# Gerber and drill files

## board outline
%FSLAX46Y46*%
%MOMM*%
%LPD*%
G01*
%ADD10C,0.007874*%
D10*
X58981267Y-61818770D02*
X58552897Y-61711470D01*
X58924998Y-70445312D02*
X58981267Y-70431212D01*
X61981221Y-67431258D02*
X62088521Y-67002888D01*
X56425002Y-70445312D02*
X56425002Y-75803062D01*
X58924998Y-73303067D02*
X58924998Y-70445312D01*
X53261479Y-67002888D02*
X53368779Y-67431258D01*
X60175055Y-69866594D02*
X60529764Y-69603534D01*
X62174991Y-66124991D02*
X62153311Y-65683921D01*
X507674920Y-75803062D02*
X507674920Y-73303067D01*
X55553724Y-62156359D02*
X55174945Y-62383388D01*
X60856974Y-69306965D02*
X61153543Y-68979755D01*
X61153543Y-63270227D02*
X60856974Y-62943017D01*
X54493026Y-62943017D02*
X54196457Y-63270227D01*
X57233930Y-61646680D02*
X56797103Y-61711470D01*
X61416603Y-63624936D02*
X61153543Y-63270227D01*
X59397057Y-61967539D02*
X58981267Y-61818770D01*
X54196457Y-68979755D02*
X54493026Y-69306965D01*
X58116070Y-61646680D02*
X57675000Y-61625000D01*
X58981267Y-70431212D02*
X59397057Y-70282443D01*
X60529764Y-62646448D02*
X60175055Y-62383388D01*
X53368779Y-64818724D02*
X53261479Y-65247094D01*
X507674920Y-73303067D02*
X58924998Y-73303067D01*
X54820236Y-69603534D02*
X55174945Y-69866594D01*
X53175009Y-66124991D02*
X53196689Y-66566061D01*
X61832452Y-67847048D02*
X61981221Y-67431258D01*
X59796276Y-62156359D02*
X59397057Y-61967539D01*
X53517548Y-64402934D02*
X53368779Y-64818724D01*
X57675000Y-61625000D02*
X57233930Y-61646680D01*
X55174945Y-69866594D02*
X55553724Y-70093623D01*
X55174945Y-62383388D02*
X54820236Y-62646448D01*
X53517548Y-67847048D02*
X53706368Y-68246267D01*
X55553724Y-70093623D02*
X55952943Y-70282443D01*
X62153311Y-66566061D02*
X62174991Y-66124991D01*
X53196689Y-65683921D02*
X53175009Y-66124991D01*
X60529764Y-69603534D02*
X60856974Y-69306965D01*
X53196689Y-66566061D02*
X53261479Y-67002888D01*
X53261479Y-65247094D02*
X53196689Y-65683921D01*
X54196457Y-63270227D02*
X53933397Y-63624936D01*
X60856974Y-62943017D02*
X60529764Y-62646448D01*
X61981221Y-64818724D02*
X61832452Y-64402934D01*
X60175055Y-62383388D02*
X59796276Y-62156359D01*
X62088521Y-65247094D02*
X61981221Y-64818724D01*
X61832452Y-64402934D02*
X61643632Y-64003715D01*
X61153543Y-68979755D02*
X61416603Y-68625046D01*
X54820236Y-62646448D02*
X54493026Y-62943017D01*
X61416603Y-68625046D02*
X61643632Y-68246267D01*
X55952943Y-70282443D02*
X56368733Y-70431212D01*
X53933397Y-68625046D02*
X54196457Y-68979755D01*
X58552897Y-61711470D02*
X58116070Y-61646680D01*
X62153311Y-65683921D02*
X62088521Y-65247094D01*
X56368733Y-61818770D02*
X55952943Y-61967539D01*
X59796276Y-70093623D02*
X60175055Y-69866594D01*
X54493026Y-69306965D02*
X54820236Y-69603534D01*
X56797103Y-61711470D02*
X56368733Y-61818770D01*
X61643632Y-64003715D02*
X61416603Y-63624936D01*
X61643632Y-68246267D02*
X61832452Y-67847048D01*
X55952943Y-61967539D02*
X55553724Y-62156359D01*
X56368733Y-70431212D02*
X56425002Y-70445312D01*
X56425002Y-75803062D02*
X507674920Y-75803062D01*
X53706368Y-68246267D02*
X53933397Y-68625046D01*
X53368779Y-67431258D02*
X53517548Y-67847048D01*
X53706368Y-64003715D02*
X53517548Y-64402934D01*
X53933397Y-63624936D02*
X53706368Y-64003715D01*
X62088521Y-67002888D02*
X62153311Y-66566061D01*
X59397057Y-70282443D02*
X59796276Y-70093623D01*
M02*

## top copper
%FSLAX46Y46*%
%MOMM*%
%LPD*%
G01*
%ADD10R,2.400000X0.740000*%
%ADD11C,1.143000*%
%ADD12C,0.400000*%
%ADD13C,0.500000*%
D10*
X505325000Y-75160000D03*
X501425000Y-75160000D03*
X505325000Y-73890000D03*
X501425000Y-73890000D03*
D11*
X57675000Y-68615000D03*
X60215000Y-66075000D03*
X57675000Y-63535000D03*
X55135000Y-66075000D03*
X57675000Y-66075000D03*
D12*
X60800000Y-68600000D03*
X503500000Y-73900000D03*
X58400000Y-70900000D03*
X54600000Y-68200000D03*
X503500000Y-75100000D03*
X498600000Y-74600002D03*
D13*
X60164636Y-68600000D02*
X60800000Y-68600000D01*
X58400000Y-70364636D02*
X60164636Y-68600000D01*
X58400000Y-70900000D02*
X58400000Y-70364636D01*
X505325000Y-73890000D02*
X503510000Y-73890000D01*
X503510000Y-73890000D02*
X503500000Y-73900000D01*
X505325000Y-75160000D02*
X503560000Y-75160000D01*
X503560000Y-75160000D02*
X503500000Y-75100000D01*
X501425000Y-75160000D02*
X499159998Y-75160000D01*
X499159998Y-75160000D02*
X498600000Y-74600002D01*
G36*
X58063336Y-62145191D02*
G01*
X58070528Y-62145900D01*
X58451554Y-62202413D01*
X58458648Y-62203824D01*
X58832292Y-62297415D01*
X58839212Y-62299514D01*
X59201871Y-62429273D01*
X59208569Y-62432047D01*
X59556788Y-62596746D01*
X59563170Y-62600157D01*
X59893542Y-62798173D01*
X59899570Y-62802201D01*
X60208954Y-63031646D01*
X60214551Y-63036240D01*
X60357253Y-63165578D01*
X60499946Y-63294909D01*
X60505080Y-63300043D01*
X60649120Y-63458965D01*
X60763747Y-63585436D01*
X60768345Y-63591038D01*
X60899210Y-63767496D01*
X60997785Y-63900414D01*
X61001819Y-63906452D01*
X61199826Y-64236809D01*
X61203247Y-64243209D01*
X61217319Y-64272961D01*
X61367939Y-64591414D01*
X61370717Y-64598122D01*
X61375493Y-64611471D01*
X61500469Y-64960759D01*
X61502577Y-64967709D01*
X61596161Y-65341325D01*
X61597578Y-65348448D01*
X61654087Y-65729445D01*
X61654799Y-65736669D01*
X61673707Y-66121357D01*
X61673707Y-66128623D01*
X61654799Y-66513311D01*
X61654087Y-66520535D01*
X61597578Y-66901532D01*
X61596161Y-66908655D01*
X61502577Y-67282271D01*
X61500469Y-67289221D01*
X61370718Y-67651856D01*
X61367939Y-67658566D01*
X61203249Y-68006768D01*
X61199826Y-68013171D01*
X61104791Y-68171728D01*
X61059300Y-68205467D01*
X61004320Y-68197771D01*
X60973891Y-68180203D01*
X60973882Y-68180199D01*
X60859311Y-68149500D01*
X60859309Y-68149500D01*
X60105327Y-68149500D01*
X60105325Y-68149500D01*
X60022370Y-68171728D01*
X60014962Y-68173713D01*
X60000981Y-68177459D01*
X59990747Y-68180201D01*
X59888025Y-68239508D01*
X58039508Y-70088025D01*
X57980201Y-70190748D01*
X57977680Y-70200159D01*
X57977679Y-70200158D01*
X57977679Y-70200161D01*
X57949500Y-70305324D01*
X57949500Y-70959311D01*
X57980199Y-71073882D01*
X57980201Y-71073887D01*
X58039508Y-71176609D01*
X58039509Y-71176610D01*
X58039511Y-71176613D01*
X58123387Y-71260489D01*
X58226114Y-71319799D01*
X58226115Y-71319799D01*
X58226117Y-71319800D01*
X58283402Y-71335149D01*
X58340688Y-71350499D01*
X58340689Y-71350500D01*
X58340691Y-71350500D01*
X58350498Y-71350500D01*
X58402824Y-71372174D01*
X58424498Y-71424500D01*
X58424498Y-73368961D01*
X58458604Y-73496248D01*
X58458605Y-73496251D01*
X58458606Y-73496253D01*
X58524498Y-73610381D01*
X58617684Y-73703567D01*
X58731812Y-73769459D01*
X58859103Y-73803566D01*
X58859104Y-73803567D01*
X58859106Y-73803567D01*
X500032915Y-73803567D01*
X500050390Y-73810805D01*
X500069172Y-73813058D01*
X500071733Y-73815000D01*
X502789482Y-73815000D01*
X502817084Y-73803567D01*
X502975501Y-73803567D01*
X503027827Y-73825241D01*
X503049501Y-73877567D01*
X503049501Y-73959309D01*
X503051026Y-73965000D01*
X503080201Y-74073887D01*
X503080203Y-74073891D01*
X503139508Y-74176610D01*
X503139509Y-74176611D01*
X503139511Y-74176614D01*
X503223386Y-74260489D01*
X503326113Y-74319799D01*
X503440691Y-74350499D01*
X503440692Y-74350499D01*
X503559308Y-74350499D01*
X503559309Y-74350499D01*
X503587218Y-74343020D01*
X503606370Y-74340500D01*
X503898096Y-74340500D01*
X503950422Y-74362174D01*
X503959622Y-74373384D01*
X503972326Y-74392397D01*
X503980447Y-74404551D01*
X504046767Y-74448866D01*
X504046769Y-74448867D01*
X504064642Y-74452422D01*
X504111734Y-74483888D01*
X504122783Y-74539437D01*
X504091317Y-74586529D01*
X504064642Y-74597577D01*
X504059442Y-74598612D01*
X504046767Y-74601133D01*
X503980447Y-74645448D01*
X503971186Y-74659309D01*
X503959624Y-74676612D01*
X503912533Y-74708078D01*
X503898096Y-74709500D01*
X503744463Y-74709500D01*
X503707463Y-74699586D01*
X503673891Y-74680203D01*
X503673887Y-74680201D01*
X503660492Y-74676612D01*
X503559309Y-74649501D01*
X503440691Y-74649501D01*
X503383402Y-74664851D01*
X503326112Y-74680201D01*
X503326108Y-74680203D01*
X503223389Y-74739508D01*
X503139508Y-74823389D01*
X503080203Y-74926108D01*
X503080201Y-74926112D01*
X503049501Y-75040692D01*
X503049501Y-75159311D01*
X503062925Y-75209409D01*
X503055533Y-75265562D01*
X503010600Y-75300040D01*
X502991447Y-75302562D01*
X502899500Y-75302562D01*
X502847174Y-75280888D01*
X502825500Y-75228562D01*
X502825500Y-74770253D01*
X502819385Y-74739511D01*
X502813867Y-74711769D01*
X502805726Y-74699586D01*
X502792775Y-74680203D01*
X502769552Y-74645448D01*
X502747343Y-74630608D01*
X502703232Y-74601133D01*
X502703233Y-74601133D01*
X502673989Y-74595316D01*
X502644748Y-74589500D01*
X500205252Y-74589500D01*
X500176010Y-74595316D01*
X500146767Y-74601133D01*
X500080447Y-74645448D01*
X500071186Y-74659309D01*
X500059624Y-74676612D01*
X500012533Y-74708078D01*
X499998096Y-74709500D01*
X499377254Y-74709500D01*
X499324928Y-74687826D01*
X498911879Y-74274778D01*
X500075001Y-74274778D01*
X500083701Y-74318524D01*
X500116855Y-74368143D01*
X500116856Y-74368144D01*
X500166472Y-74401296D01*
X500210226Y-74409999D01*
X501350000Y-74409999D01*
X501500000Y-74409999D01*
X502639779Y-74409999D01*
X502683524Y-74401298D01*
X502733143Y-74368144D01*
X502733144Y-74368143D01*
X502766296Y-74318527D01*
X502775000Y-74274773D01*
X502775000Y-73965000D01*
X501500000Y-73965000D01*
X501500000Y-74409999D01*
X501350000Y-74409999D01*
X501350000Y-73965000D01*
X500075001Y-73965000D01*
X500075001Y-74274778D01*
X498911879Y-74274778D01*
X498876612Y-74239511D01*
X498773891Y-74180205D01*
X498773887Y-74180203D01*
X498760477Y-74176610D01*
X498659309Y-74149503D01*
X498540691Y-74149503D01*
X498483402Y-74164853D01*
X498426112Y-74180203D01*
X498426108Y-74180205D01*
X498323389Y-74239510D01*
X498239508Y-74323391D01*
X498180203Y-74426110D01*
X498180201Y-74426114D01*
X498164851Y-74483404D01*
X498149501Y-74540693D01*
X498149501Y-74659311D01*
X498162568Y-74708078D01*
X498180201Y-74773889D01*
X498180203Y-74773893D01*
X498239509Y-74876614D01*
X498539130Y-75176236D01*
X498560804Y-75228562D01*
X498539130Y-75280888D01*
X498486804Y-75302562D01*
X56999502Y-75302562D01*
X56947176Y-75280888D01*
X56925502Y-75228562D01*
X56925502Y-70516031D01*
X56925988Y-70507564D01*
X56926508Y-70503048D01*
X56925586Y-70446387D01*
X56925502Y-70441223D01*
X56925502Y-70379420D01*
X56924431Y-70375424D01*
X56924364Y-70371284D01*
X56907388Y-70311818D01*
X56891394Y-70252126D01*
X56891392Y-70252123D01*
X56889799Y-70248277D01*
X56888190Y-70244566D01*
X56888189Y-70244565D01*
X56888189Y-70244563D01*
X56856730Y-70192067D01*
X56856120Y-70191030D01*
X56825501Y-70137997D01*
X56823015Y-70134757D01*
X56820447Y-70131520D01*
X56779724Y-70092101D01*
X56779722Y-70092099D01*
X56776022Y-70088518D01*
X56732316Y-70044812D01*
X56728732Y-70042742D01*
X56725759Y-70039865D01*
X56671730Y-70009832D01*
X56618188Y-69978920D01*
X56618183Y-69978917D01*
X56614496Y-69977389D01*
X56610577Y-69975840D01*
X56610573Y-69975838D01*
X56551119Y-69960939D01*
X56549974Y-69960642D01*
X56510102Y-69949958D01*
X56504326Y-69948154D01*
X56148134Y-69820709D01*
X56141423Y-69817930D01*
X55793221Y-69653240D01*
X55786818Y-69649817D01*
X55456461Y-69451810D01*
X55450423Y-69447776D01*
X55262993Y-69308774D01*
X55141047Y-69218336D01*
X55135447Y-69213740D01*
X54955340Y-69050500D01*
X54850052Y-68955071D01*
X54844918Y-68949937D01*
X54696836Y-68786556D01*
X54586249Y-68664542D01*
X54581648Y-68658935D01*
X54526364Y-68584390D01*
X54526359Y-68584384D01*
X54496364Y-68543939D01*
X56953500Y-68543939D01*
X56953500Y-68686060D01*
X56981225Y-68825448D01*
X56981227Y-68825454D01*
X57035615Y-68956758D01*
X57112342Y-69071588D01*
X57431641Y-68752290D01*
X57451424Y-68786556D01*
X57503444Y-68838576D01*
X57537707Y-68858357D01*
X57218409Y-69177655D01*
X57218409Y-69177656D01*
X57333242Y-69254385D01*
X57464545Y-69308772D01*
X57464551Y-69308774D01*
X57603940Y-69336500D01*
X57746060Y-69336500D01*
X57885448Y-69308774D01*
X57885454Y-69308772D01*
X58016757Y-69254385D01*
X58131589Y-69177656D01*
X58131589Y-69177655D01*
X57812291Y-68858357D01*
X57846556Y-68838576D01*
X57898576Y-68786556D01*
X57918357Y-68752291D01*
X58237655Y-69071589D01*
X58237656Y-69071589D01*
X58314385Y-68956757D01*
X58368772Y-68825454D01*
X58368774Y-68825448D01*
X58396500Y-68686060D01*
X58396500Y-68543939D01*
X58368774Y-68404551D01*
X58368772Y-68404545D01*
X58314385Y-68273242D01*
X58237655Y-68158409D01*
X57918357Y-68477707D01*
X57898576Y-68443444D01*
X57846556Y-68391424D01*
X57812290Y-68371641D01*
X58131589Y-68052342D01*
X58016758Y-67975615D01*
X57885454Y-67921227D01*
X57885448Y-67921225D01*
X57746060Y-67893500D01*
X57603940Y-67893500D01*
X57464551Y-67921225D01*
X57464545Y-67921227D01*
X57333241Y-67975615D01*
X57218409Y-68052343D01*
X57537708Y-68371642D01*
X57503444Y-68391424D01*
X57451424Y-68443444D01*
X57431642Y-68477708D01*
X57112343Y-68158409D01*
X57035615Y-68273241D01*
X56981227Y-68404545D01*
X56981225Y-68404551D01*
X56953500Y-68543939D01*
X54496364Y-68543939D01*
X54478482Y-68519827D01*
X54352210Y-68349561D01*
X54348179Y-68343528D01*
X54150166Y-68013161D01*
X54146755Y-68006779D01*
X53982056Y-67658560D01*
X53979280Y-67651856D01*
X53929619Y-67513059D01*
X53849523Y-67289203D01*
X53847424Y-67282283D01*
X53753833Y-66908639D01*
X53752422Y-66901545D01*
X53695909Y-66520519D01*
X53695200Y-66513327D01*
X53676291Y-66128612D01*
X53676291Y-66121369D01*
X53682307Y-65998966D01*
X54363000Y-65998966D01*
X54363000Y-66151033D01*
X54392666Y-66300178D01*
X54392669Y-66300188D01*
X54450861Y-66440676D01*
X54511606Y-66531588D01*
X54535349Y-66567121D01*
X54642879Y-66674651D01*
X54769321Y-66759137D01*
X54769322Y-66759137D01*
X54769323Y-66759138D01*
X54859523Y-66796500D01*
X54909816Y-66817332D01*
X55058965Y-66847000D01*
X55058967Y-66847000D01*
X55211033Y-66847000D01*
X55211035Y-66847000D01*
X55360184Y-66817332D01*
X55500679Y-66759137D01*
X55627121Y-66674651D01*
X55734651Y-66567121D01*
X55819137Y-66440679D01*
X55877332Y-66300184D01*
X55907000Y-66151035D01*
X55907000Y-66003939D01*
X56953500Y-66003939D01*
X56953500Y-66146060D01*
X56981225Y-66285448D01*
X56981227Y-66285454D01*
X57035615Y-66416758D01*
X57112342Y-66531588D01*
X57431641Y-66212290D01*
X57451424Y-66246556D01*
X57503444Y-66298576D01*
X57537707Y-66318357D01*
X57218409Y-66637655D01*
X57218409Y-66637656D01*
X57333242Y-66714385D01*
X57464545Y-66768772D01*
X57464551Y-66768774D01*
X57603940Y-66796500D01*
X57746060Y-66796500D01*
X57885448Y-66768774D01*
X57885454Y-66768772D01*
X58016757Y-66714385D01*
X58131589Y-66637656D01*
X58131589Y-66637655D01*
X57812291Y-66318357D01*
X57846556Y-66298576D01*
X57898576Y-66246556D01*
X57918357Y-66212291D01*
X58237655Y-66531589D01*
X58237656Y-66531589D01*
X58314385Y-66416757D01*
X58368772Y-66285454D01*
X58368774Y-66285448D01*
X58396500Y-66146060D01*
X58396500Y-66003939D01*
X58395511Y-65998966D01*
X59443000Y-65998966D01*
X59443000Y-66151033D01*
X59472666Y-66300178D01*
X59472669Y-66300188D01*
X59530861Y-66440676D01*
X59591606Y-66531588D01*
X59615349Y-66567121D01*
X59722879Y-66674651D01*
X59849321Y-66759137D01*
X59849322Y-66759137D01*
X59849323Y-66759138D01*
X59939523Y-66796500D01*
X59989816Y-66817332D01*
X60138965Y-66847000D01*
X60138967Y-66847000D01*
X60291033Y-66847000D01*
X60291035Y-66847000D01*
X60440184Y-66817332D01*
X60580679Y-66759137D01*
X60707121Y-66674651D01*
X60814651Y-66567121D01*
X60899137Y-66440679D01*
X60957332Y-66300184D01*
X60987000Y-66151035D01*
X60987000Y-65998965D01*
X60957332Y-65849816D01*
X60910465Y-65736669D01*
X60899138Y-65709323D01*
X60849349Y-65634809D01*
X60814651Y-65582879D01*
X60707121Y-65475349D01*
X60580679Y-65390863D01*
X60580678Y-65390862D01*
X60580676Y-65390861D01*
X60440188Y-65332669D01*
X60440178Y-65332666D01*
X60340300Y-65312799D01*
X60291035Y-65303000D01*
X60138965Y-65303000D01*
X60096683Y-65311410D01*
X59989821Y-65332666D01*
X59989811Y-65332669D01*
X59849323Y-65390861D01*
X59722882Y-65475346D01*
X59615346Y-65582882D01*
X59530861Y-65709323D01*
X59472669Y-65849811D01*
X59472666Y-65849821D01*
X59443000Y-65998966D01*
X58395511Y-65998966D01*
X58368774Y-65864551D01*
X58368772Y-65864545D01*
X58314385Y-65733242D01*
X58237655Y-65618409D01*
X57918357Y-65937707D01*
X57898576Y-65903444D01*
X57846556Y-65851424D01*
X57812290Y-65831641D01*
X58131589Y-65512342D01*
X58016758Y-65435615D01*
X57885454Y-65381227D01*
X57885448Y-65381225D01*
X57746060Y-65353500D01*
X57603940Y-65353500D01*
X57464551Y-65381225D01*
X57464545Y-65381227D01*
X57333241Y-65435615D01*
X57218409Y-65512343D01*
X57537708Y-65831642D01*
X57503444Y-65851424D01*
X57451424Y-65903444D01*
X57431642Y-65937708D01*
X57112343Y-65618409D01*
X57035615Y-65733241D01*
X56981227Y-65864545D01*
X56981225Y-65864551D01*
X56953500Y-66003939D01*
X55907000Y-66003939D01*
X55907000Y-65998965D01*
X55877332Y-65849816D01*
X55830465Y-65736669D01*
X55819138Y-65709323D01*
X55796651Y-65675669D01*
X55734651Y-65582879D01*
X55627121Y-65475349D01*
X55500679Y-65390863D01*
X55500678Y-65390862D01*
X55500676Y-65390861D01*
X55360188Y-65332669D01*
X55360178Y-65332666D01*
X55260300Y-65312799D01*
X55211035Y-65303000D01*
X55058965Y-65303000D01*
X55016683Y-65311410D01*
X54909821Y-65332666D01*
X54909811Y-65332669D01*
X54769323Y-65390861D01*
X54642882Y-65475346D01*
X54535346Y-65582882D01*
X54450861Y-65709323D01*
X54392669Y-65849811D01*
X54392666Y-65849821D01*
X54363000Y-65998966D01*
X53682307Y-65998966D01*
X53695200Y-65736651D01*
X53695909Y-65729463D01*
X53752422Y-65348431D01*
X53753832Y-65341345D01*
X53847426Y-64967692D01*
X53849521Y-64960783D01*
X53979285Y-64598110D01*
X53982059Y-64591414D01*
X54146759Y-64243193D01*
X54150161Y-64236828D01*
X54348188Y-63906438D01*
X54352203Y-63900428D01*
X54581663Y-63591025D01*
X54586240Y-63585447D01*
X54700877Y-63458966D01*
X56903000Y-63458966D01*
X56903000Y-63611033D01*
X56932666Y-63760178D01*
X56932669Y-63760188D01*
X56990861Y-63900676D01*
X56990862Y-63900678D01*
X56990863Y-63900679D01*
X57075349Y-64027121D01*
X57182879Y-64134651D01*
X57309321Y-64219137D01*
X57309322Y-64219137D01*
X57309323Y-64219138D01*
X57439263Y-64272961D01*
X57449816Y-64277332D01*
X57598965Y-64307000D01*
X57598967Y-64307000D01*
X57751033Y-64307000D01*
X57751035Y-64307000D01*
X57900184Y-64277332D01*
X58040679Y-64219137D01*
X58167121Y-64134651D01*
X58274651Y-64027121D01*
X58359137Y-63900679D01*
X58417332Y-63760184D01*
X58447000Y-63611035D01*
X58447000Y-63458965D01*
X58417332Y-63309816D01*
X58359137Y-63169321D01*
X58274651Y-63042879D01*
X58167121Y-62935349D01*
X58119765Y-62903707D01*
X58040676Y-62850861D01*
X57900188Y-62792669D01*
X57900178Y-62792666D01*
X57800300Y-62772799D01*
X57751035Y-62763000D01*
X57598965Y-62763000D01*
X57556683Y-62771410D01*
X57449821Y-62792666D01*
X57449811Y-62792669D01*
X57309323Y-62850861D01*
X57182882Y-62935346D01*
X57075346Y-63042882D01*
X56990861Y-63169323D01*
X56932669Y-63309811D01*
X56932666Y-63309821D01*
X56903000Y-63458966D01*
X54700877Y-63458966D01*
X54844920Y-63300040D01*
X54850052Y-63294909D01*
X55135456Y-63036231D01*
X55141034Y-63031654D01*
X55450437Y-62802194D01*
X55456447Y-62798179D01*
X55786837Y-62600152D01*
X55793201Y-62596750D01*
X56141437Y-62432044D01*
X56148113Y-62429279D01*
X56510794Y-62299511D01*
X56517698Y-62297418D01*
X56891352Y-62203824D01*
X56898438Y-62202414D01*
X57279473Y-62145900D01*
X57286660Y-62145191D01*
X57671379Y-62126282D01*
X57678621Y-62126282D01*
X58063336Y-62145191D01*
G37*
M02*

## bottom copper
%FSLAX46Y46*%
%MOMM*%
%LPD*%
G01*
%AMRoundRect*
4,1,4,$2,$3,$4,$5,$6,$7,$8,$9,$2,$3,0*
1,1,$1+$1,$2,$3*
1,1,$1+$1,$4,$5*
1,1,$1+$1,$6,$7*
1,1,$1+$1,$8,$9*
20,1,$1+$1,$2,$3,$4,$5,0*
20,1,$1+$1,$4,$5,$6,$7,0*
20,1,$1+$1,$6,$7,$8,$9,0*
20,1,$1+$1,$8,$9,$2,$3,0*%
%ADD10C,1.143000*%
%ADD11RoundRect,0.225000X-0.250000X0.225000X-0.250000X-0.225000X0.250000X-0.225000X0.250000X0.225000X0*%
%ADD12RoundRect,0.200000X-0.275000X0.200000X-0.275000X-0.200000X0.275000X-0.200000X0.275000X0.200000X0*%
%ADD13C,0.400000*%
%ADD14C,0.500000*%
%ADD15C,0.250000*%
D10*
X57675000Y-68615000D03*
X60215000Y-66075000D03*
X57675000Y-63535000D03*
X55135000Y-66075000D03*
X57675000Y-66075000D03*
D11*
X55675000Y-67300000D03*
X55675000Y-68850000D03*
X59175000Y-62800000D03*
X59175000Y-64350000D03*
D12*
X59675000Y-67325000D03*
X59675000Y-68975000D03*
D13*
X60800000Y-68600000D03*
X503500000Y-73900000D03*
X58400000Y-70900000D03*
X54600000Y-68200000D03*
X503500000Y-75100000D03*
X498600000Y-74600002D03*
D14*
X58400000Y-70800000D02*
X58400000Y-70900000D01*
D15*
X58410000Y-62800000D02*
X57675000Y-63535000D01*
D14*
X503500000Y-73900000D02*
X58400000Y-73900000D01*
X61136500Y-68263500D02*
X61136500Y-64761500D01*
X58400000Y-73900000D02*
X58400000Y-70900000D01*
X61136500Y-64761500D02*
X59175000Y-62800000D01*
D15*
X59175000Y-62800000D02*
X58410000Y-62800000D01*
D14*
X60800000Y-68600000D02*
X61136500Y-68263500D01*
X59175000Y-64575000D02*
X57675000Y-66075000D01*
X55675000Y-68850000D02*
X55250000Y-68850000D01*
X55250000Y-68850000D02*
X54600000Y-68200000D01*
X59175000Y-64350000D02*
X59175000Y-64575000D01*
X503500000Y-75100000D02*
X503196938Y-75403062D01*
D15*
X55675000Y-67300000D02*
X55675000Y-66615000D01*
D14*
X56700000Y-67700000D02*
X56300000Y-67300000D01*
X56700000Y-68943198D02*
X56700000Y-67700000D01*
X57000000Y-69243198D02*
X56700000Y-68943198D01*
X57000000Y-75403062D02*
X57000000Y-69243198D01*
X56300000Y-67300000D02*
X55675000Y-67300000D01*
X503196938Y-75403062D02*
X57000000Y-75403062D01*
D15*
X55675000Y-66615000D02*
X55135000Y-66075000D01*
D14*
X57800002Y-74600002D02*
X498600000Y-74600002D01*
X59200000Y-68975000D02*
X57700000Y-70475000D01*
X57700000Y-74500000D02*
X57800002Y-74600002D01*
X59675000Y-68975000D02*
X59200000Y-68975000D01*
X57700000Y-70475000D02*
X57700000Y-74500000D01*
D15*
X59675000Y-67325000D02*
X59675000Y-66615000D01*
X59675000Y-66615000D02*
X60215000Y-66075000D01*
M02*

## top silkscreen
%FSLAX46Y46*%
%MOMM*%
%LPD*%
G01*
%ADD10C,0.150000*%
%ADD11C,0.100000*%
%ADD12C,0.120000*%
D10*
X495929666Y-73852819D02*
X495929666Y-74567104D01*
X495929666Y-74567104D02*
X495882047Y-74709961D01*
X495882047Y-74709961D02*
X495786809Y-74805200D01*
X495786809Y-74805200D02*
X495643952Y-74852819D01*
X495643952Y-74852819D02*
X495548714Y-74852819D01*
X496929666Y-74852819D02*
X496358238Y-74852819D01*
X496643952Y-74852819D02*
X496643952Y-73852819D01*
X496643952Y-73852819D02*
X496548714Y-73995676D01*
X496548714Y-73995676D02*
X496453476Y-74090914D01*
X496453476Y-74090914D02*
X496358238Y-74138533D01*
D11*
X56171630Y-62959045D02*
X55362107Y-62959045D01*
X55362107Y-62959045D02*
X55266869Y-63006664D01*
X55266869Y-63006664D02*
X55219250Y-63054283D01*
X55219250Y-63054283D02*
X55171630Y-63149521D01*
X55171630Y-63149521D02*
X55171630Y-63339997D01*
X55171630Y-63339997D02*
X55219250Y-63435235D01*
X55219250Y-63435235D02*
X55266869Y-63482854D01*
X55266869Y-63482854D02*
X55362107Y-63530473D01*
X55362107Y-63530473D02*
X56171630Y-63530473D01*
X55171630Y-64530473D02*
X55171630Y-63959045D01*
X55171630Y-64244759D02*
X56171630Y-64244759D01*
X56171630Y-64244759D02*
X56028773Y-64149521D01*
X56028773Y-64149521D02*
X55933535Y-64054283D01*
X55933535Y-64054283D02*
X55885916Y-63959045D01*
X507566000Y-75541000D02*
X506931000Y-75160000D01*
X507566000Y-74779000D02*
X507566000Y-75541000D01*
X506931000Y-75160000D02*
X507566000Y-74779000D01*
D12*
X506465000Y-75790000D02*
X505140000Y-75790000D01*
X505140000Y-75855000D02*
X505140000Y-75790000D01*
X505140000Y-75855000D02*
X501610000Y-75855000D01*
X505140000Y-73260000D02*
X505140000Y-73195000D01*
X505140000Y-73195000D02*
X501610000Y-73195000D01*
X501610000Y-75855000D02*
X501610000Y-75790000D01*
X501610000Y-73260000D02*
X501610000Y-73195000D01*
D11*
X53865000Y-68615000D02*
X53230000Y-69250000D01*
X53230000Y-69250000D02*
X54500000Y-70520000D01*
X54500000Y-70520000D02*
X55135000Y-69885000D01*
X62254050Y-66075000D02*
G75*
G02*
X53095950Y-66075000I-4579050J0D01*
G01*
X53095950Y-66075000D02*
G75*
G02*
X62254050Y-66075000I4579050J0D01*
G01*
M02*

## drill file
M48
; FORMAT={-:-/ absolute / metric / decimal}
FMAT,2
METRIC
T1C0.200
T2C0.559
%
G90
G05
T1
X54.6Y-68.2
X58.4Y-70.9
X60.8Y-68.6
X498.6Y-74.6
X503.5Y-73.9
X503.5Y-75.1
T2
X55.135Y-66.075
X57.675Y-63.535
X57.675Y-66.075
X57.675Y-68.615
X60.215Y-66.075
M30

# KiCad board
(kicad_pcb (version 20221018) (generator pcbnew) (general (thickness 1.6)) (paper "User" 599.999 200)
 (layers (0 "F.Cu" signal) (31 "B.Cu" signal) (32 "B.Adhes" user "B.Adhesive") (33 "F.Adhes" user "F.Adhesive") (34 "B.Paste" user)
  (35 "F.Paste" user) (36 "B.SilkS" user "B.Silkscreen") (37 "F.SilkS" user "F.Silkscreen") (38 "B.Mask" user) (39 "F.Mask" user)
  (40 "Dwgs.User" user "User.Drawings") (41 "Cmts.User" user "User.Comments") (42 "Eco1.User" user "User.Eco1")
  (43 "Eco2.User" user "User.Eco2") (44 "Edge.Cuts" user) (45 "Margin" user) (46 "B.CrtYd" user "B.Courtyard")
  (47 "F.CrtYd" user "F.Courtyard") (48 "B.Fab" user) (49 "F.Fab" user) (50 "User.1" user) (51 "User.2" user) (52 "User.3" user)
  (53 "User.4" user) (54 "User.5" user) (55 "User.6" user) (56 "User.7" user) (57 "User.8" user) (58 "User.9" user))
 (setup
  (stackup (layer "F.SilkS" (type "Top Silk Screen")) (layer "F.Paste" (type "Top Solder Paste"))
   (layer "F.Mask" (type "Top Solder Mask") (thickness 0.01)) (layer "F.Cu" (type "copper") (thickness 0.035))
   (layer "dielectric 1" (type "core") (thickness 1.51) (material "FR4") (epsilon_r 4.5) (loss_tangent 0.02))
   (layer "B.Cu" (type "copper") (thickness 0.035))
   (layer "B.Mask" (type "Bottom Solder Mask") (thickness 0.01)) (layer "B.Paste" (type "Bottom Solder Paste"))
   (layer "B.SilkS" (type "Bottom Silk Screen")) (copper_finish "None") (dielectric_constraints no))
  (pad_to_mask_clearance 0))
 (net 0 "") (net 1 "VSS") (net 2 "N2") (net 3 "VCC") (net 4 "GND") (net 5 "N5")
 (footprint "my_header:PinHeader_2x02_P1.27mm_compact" (layer "F.Cu") (at 503.375 74.525 180)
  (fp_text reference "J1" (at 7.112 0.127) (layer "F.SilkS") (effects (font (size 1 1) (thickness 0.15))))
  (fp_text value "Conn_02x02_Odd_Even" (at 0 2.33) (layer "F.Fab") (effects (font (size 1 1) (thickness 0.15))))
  (fp_line (start -4.191 -1.016) (end -3.556 -0.635) (stroke (width 0.1) (type default)) (layer "F.SilkS"))
  (fp_line (start -4.191 -0.254) (end -4.191 -1.016) (stroke (width 0.1) (type default)) (layer "F.SilkS"))
  (fp_line (start -3.556 -0.635) (end -4.191 -0.254) (stroke (width 0.1) (type default)) (layer "F.SilkS"))
  (fp_line (start -3.09 -1.265) (end -1.765 -1.265) (stroke (width 0.12) (type solid)) (layer "F.SilkS"))
  (fp_line (start -1.765 -1.33) (end -1.765 -1.265) (stroke (width 0.12) (type solid)) (layer "F.SilkS"))
  (fp_line (start -1.765 -1.33) (end 1.765 -1.33) (stroke (width 0.12) (type solid)) (layer "F.SilkS"))
  (fp_line (start -1.765 1.265) (end -1.765 1.33) (stroke (width 0.12) (type solid)) (layer "F.SilkS"))
  (fp_line (start -1.765 1.33) (end 1.765 1.33) (stroke (width 0.12) (type solid)) (layer "F.SilkS"))
  (fp_line (start 1.765 -1.33) (end 1.765 -1.265) (stroke (width 0.12) (type solid)) (layer "F.SilkS"))
  (fp_line (start 1.765 1.265) (end 1.765 1.33) (stroke (width 0.12) (type solid)) (layer "F.SilkS"))
  (pad "1" smd rect (at -1.95 -0.635 180) (size 2.4 0.74) (layers "F.Cu" "F.Paste" "F.Mask") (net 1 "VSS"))
  (pad "2" smd rect (at 1.95 -0.635 180) (size 2.4 0.74) (layers "F.Cu" "F.Paste" "F.Mask") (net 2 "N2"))
  (pad "3" smd rect (at -1.95 0.635 180) (size 2.4 0.74) (layers "F.Cu" "F.Paste" "F.Mask") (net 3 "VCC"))
  (pad "4" smd rect (at 1.95 0.635 180) (size 2.4 0.74) (layers "F.Cu" "F.Paste" "F.Mask") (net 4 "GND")))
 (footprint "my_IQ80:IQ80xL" (layer "F.Cu") (at 57.675 63.535 -90)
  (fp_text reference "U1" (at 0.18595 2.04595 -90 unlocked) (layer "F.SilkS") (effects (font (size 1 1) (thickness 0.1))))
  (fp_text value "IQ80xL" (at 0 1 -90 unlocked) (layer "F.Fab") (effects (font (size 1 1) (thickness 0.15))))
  (fp_line (start 5.08 3.81) (end 5.715 4.445) (stroke (width 0.1) (type default)) (layer "F.SilkS"))
  (fp_line (start 5.715 4.445) (end 6.985 3.175) (stroke (width 0.1) (type default)) (layer "F.SilkS"))
  (fp_line (start 6.985 3.175) (end 6.35 2.54) (stroke (width 0.1) (type default)) (layer "F.SilkS"))
  (fp_circle (center 2.54 0) (end 6.35 2.54) (stroke (width 0.1) (type default)) (fill none) (layer "F.SilkS"))
  (pad "1" thru_hole circle (at 5.08 0 270) (size 1.143 1.143) (drill 0.5588) (layers "*.Cu" "*.Mask") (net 4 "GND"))
  (pad "2" thru_hole circle (at 2.54 -2.54 270) (size 1.143 1.143) (drill 0.5588) (layers "*.Cu" "*.Mask") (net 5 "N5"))
  (pad "3" thru_hole circle (at 0 0 270) (size 1.143 1.143) (drill 0.5588) (layers "*.Cu" "*.Mask") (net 3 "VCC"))
  (pad "4" thru_hole circle (at 2.54 2.54 270) (size 1.143 1.143) (drill 0.5588) (layers "*.Cu" "*.Mask") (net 1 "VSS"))
  (pad "5" thru_hole circle (at 2.54 0 270) (size 1.143 1.143) (drill 0.5588) (layers "*.Cu" "*.Mask") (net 4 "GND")))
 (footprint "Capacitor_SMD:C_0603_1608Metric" (layer "B.Cu") (at 55.675 68.075 -90)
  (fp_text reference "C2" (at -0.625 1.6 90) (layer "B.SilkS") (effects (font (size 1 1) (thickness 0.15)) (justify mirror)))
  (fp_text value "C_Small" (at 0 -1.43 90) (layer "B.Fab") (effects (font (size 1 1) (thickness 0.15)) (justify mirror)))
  (pad "1" smd roundrect (at -0.775 0 270) (size 0.9 0.95) (layers "B.Cu" "B.Paste" "B.Mask") (roundrect_rratio 0.25) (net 1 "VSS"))
  (pad "2" smd roundrect (at 0.775 0 270) (size 0.9 0.95) (layers "B.Cu" "B.Paste" "B.Mask") (roundrect_rratio 0.25) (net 4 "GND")))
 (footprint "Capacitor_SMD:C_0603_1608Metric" (layer "B.Cu") (at 59.175 63.575 -90)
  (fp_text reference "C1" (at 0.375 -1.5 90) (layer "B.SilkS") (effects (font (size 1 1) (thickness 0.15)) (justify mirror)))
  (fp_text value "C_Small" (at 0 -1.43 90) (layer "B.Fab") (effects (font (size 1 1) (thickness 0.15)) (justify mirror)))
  (pad "1" smd roundrect (at -0.775 0 270) (size 0.9 0.95) (layers "B.Cu" "B.Paste" "B.Mask") (roundrect_rratio 0.25) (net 3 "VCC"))
  (pad "2" smd roundrect (at 0.775 0 270) (size 0.9 0.95) (layers "B.Cu" "B.Paste" "B.Mask") (roundrect_rratio 0.25) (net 4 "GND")))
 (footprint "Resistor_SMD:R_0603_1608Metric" (layer "B.Cu") (at 59.675 68.15 -90)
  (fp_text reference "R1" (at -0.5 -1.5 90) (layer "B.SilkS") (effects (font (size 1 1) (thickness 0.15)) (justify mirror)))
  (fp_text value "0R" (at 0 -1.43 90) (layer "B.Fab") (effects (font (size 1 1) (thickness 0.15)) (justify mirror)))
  (pad "1" smd roundrect (at -0.825 0 270) (size 0.8 0.95) (layers "B.Cu" "B.Paste" "B.Mask") (roundrect_rratio 0.25) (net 5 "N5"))
  (pad "2" smd roundrect (at 0.825 0 270) (size 0.8 0.95) (layers "B.Cu" "B.Paste" "B.Mask") (roundrect_rratio 0.25) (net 2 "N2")))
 (gr_line (start 58.981267 61.81877) (end 58.552897 61.71147) (stroke (width 0.007874) (type solid)) (layer "Edge.Cuts"))
 (gr_line (start 58.924998 70.445312) (end 58.981267 70.431212) (stroke (width 0.007874) (type solid)) (layer "Edge.Cuts"))
 (gr_line (start 61.981221 67.431258) (end 62.088521 67.002888) (stroke (width 0.007874) (type solid)) (layer "Edge.Cuts"))
 (gr_line (start 56.425002 70.445312) (end 56.425002 75.803062) (stroke (width 0.007874) (type solid)) (layer "Edge.Cuts"))
 (gr_line (start 58.924998 73.303067) (end 58.924998 70.445312) (stroke (width 0.007874) (type solid)) (layer "Edge.Cuts"))
 (gr_line (start 53.261479 67.002888) (end 53.368779 67.431258) (stroke (width 0.007874) (type solid)) (layer "Edge.Cuts"))
 (gr_line (start 60.175055 69.866594) (end 60.529764 69.603534) (stroke (width 0.007874) (type solid)) (layer "Edge.Cuts"))
 (gr_line (start 62.174991 66.124991) (end 62.153311 65.683921) (stroke (width 0.007874) (type solid)) (layer "Edge.Cuts"))
 (gr_line (start 507.67492 75.803062) (end 507.67492 73.303067) (stroke (width 0.007874) (type solid)) (layer "Edge.Cuts"))
 (gr_line (start 55.553724 62.156359) (end 55.174945 62.383388) (stroke (width 0.007874) (type solid)) (layer "Edge.Cuts"))
 (gr_line (start 60.856974 69.306965) (end 61.153543 68.979755) (stroke (width 0.007874) (type solid)) (layer "Edge.Cuts"))
 (gr_line (start 61.153543 63.270227) (end 60.856974 62.943017) (stroke (width 0.007874) (type solid)) (layer "Edge.Cuts"))
 (gr_line (start 54.493026 62.943017) (end 54.196457 63.270227) (stroke (width 0.007874) (type solid)) (layer "Edge.Cuts"))
 (gr_line (start 57.23393 61.64668) (end 56.797103 61.71147) (stroke (width 0.007874) (type solid)) (layer "Edge.Cuts"))
 (gr_line (start 61.416603 63.624936) (end 61.153543 63.270227) (stroke (width 0.007874) (type solid)) (layer "Edge.Cuts"))
 (gr_line (start 59.397057 61.967539) (end 58.981267 61.81877) (stroke (width 0.007874) (type solid)) (layer "Edge.Cuts"))
 (gr_line (start 54.196457 68.979755) (end 54.493026 69.306965) (stroke (width 0.007874) (type solid)) (layer "Edge.Cuts"))
 (gr_line (start 58.11607 61.64668) (end 57.675 61.625) (stroke (width 0.007874) (type solid)) (layer "Edge.Cuts"))
 (gr_line (start 58.981267 70.431212) (end 59.397057 70.282443) (stroke (width 0.007874) (type solid)) (layer "Edge.Cuts"))
 (gr_line (start 60.529764 62.646448) (end 60.175055 62.383388) (stroke (width 0.007874) (type solid)) (layer "Edge.Cuts"))
 (gr_line (start 53.368779 64.818724) (end 53.261479 65.247094) (stroke (width 0.007874) (type solid)) (layer "Edge.Cuts"))
 (gr_line (start 507.67492 73.303067) (end 58.924998 73.303067) (stroke (width 0.007874) (type solid)) (layer "Edge.Cuts"))
 (gr_line (start 54.820236 69.603534) (end 55.174945 69.866594) (stroke (width 0.007874) (type solid)) (layer "Edge.Cuts"))
 (gr_line (start 53.175009 66.124991) (end 53.196689 66.566061) (stroke (width 0.007874) (type solid)) (layer "Edge.Cuts"))
 (gr_line (start 61.832452 67.847048) (end 61.981221 67.431258) (stroke (width 0.007874) (type solid)) (layer "Edge.Cuts"))
 (gr_line (start 59.796276 62.156359) (end 59.397057 61.967539) (stroke (width 0.007874) (type solid)) (layer "Edge.Cuts"))
 (gr_line (start 53.517548 64.402934) (end 53.368779 64.818724) (stroke (width 0.007874) (type solid)) (layer "Edge.Cuts"))
 (gr_line (start 57.675 61.625) (end 57.23393 61.64668) (stroke (width 0.007874) (type solid)) (layer "Edge.Cuts"))
 (gr_line (start 55.174945 69.866594) (end 55.553724 70.093623) (stroke (width 0.007874) (type solid)) (layer "Edge.Cuts"))
 (gr_line (start 55.174945 62.383388) (end 54.820236 62.646448) (stroke (width 0.007874) (type solid)) (layer "Edge.Cuts"))
 (gr_line (start 53.517548 67.847048) (end 53.706368 68.246267) (stroke (width 0.007874) (type solid)) (layer "Edge.Cuts"))
 (gr_line (start 55.553724 70.093623) (end 55.952943 70.282443) (stroke (width 0.007874) (type solid)) (layer "Edge.Cuts"))
 (gr_line (start 62.153311 66.566061) (end 62.174991 66.124991) (stroke (width 0.007874) (type solid)) (layer "Edge.Cuts"))
 (gr_line (start 53.196689 65.683921) (end 53.175009 66.124991) (stroke (width 0.007874) (type solid)) (layer "Edge.Cuts"))
 (gr_line (start 60.529764 69.603534) (end 60.856974 69.306965) (stroke (width 0.007874) (type solid)) (layer "Edge.Cuts"))
 (gr_line (start 53.196689 66.566061) (end 53.261479 67.002888) (stroke (width 0.007874) (type solid)) (layer "Edge.Cuts"))
 (gr_line (start 53.261479 65.247094) (end 53.196689 65.683921) (stroke (width 0.007874) (type solid)) (layer "Edge.Cuts"))
 (gr_line (start 54.196457 63.270227) (end 53.933397 63.624936) (stroke (width 0.007874) (type solid)) (layer "Edge.Cuts"))
 (gr_line (start 60.856974 62.943017) (end 60.529764 62.646448) (stroke (width 0.007874) (type solid)) (layer "Edge.Cuts"))
 (gr_line (start 61.981221 64.818724) (end 61.832452 64.402934) (stroke (width 0.007874) (type solid)) (layer "Edge.Cuts"))
 (gr_line (start 60.175055 62.383388) (end 59.796276 62.156359) (stroke (width 0.007874) (type solid)) (layer "Edge.Cuts"))
 (gr_line (start 62.088521 65.247094) (end 61.981221 64.818724) (stroke (width 0.007874) (type solid)) (layer "Edge.Cuts"))
 (gr_line (start 61.832452 64.402934) (end 61.643632 64.003715) (stroke (width 0.007874) (type solid)) (layer "Edge.Cuts"))
 (gr_line (start 61.153543 68.979755) (end 61.416603 68.625046) (stroke (width 0.007874) (type solid)) (layer "Edge.Cuts"))
 (gr_line (start 54.820236 62.646448) (end 54.493026 62.943017) (stroke (width 0.007874) (type solid)) (layer "Edge.Cuts"))
 (gr_line (start 61.416603 68.625046) (end 61.643632 68.246267) (stroke (width 0.007874) (type solid)) (layer "Edge.Cuts"))
 (gr_line (start 55.952943 70.282443) (end 56.368733 70.431212) (stroke (width 0.007874) (type solid)) (layer "Edge.Cuts"))
 (gr_line (start 53.933397 68.625046) (end 54.196457 68.979755) (stroke (width 0.007874) (type solid)) (layer "Edge.Cuts"))
 (gr_line (start 58.552897 61.71147) (end 58.11607 61.64668) (stroke (width 0.007874) (type solid)) (layer "Edge.Cuts"))
 (gr_line (start 62.153311 65.683921) (end 62.088521 65.247094) (stroke (width 0.007874) (type solid)) (layer "Edge.Cuts"))
 (gr_line (start 56.368733 61.81877) (end 55.952943 61.967539) (stroke (width 0.007874) (type solid)) (layer "Edge.Cuts"))
 (gr_line (start 59.796276 70.093623) (end 60.175055 69.866594) (stroke (width 0.007874) (type solid)) (layer "Edge.Cuts"))
 (gr_line (start 54.493026 69.306965) (end 54.820236 69.603534) (stroke (width 0.007874) (type solid)) (layer "Edge.Cuts"))
 (gr_line (start 56.797103 61.71147) (end 56.368733 61.81877) (stroke (width 0.007874) (type solid)) (layer "Edge.Cuts"))
 (gr_line (start 61.643632 64.003715) (end 61.416603 63.624936) (stroke (width 0.007874) (type solid)) (layer "Edge.Cuts"))
 (gr_line (start 61.643632 68.246267) (end 61.832452 67.847048) (stroke (width 0.007874) (type solid)) (layer "Edge.Cuts"))
 (gr_line (start 55.952943 61.967539) (end 55.553724 62.156359) (stroke (width 0.007874) (type solid)) (layer "Edge.Cuts"))
 (gr_line (start 56.368733 70.431212) (end 56.425002 70.445312) (stroke (width 0.007874) (type solid)) (layer "Edge.Cuts"))
 (gr_line (start 56.425002 75.803062) (end 507.67492 75.803062) (stroke (width 0.007874) (type solid)) (layer "Edge.Cuts"))
 (gr_line (start 53.706368 68.246267) (end 53.933397 68.625046) (stroke (width 0.007874) (type solid)) (layer "Edge.Cuts"))
 (gr_line (start 53.368779 67.431258) (end 53.517548 67.847048) (stroke (width 0.007874) (type solid)) (layer "Edge.Cuts"))
 (gr_line (start 53.706368 64.003715) (end 53.517548 64.402934) (stroke (width 0.007874) (type solid)) (layer "Edge.Cuts"))
 (gr_line (start 53.933397 63.624936) (end 53.706368 64.003715) (stroke (width 0.007874) (type solid)) (layer "Edge.Cuts"))
 (gr_line (start 62.088521 67.002888) (end 62.153311 66.566061) (stroke (width 0.007874) (type solid)) (layer "Edge.Cuts"))
 (gr_line (start 59.397057 70.282443) (end 59.796276 70.093623) (stroke (width 0.007874) (type solid)) (layer "Edge.Cuts"))
 (segment (start 60.164636 68.6) (end 60.8 68.6) (width 0.5) (layer "F.Cu") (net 3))
 (segment (start 58.4 70.364636) (end 60.164636 68.6) (width 0.5) (layer "F.Cu") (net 3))
 (segment (start 58.4 70.9) (end 58.4 70.364636) (width 0.5) (layer "F.Cu") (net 3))
 (segment (start 505.325 73.89) (end 503.51 73.89) (width 0.5) (layer "F.Cu") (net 3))
 (segment (start 503.51 73.89) (end 503.5 73.9) (width 0.5) (layer "F.Cu") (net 3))
 (via (at 60.8 68.6) (size 0.4) (drill 0.2) (layers "F.Cu" "B.Cu") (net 3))
 (via (at 503.5 73.9) (size 0.4) (drill 0.2) (layers "F.Cu" "B.Cu") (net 3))
 (via (at 58.4 70.9) (size 0.4) (drill 0.2) (layers "F.Cu" "B.Cu") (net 3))
 (segment (start 58.4 70.8) (end 58.4 70.9) (width 0.5) (layer "B.Cu") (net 3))
 (segment (start 58.41 62.8) (end 57.675 63.535) (width 0.25) (layer "B.Cu") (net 3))
 (segment (start 503.5 73.9) (end 58.4 73.9) (width 0.5) (layer "B.Cu") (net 3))
 (segment (start 61.1365 68.2635) (end 61.1365 64.7615) (width 0.5) (layer "B.Cu") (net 3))
 (segment (start 58.4 73.9) (end 58.4 70.9) (width 0.5) (layer "B.Cu") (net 3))
 (segment (start 61.1365 64.7615) (end 59.175 62.8) (width 0.5) (layer "B.Cu") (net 3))
 (segment (start 59.175 62.8) (end 58.41 62.8) (width 0.25) (layer "B.Cu") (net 3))
 (segment (start 60.8 68.6) (end 61.1365 68.2635) (width 0.5) (layer "B.Cu") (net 3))
 (via (at 54.6 68.2) (size 0.4) (drill 0.2) (layers "F.Cu" "B.Cu") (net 4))
 (segment (start 59.175 64.575) (end 57.675 66.075) (width 0.5) (layer "B.Cu") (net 4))
 (segment (start 55.675 68.85) (end 55.25 68.85) (width 0.5) (layer "B.Cu") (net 4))
 (segment (start 55.25 68.85) (end 54.6 68.2) (width 0.5) (layer "B.Cu") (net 4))
 (segment (start 59.175 64.35) (end 59.175 64.575) (width 0.5) (layer "B.Cu") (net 4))
 (segment (start 505.325 75.16) (end 503.56 75.16) (width 0.5) (layer "F.Cu") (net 1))
 (segment (start 503.56 75.16) (end 503.5 75.1) (width 0.5) (layer "F.Cu") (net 1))
 (via (at 503.5 75.1) (size 0.4) (drill 0.2) (layers "F.Cu" "B.Cu") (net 1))
 (segment (start 503.5 75.1) (end 503.196938 75.403062) (width 0.5) (layer "B.Cu") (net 1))
 (segment (start 55.675 67.3) (end 55.675 66.615) (width 0.25) (layer "B.Cu") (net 1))
 (segment (start 56.7 67.7) (end 56.3 67.3) (width 0.5) (layer "B.Cu") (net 1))
 (segment (start 56.7 68.943198) (end 56.7 67.7) (width 0.5) (layer "B.Cu") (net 1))
 (segment (start 57 69.243198) (end 56.7 68.943198) (width 0.5) (layer "B.Cu") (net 1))
 (segment (start 57 75.403062) (end 57 69.243198) (width 0.5) (layer "B.Cu") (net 1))
 (segment (start 56.3 67.3) (end 55.675 67.3) (width 0.5) (layer "B.Cu") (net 1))
 (segment (start 503.196938 75.403062) (end 57 75.403062) (width 0.5) (layer "B.Cu") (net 1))
 (segment (start 55.675 66.615) (end 55.135 66.075) (width 0.25) (layer "B.Cu") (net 1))
 (segment (start 501.425 75.16) (end 499.159998 75.16) (width 0.5) (layer "F.Cu") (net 2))
 (segment (start 499.159998 75.16) (end 498.6 74.600002) (width 0.5) (layer "F.Cu") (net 2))
 (via (at 498.6 74.600002) (size 0.4) (drill 0.2) (layers "F.Cu" "B.Cu") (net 2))
 (segment (start 57.800002 74.600002) (end 498.6 74.600002) (width 0.5) (layer "B.Cu") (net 2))
 (segment (start 59.2 68.975) (end 57.7 70.475) (width 0.5) (layer "B.Cu") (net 2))
 (segment (start 57.7 74.5) (end 57.800002 74.600002) (width 0.5) (layer "B.Cu") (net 2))
 (segment (start 59.675 68.975) (end 59.2 68.975) (width 0.5) (layer "B.Cu") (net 2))
 (segment (start 57.7 70.475) (end 57.7 74.5) (width 0.5) (layer "B.Cu") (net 2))
 (segment (start 59.675 67.325) (end 59.675 66.615) (width 0.25) (layer "B.Cu") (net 5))
 (segment (start 59.675 66.615) (end 60.215 66.075) (width 0.25) (layer "B.Cu") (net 5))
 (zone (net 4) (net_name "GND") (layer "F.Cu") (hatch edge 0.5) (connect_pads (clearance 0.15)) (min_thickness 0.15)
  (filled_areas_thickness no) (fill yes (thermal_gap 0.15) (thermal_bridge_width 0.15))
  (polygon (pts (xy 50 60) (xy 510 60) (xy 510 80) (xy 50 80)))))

